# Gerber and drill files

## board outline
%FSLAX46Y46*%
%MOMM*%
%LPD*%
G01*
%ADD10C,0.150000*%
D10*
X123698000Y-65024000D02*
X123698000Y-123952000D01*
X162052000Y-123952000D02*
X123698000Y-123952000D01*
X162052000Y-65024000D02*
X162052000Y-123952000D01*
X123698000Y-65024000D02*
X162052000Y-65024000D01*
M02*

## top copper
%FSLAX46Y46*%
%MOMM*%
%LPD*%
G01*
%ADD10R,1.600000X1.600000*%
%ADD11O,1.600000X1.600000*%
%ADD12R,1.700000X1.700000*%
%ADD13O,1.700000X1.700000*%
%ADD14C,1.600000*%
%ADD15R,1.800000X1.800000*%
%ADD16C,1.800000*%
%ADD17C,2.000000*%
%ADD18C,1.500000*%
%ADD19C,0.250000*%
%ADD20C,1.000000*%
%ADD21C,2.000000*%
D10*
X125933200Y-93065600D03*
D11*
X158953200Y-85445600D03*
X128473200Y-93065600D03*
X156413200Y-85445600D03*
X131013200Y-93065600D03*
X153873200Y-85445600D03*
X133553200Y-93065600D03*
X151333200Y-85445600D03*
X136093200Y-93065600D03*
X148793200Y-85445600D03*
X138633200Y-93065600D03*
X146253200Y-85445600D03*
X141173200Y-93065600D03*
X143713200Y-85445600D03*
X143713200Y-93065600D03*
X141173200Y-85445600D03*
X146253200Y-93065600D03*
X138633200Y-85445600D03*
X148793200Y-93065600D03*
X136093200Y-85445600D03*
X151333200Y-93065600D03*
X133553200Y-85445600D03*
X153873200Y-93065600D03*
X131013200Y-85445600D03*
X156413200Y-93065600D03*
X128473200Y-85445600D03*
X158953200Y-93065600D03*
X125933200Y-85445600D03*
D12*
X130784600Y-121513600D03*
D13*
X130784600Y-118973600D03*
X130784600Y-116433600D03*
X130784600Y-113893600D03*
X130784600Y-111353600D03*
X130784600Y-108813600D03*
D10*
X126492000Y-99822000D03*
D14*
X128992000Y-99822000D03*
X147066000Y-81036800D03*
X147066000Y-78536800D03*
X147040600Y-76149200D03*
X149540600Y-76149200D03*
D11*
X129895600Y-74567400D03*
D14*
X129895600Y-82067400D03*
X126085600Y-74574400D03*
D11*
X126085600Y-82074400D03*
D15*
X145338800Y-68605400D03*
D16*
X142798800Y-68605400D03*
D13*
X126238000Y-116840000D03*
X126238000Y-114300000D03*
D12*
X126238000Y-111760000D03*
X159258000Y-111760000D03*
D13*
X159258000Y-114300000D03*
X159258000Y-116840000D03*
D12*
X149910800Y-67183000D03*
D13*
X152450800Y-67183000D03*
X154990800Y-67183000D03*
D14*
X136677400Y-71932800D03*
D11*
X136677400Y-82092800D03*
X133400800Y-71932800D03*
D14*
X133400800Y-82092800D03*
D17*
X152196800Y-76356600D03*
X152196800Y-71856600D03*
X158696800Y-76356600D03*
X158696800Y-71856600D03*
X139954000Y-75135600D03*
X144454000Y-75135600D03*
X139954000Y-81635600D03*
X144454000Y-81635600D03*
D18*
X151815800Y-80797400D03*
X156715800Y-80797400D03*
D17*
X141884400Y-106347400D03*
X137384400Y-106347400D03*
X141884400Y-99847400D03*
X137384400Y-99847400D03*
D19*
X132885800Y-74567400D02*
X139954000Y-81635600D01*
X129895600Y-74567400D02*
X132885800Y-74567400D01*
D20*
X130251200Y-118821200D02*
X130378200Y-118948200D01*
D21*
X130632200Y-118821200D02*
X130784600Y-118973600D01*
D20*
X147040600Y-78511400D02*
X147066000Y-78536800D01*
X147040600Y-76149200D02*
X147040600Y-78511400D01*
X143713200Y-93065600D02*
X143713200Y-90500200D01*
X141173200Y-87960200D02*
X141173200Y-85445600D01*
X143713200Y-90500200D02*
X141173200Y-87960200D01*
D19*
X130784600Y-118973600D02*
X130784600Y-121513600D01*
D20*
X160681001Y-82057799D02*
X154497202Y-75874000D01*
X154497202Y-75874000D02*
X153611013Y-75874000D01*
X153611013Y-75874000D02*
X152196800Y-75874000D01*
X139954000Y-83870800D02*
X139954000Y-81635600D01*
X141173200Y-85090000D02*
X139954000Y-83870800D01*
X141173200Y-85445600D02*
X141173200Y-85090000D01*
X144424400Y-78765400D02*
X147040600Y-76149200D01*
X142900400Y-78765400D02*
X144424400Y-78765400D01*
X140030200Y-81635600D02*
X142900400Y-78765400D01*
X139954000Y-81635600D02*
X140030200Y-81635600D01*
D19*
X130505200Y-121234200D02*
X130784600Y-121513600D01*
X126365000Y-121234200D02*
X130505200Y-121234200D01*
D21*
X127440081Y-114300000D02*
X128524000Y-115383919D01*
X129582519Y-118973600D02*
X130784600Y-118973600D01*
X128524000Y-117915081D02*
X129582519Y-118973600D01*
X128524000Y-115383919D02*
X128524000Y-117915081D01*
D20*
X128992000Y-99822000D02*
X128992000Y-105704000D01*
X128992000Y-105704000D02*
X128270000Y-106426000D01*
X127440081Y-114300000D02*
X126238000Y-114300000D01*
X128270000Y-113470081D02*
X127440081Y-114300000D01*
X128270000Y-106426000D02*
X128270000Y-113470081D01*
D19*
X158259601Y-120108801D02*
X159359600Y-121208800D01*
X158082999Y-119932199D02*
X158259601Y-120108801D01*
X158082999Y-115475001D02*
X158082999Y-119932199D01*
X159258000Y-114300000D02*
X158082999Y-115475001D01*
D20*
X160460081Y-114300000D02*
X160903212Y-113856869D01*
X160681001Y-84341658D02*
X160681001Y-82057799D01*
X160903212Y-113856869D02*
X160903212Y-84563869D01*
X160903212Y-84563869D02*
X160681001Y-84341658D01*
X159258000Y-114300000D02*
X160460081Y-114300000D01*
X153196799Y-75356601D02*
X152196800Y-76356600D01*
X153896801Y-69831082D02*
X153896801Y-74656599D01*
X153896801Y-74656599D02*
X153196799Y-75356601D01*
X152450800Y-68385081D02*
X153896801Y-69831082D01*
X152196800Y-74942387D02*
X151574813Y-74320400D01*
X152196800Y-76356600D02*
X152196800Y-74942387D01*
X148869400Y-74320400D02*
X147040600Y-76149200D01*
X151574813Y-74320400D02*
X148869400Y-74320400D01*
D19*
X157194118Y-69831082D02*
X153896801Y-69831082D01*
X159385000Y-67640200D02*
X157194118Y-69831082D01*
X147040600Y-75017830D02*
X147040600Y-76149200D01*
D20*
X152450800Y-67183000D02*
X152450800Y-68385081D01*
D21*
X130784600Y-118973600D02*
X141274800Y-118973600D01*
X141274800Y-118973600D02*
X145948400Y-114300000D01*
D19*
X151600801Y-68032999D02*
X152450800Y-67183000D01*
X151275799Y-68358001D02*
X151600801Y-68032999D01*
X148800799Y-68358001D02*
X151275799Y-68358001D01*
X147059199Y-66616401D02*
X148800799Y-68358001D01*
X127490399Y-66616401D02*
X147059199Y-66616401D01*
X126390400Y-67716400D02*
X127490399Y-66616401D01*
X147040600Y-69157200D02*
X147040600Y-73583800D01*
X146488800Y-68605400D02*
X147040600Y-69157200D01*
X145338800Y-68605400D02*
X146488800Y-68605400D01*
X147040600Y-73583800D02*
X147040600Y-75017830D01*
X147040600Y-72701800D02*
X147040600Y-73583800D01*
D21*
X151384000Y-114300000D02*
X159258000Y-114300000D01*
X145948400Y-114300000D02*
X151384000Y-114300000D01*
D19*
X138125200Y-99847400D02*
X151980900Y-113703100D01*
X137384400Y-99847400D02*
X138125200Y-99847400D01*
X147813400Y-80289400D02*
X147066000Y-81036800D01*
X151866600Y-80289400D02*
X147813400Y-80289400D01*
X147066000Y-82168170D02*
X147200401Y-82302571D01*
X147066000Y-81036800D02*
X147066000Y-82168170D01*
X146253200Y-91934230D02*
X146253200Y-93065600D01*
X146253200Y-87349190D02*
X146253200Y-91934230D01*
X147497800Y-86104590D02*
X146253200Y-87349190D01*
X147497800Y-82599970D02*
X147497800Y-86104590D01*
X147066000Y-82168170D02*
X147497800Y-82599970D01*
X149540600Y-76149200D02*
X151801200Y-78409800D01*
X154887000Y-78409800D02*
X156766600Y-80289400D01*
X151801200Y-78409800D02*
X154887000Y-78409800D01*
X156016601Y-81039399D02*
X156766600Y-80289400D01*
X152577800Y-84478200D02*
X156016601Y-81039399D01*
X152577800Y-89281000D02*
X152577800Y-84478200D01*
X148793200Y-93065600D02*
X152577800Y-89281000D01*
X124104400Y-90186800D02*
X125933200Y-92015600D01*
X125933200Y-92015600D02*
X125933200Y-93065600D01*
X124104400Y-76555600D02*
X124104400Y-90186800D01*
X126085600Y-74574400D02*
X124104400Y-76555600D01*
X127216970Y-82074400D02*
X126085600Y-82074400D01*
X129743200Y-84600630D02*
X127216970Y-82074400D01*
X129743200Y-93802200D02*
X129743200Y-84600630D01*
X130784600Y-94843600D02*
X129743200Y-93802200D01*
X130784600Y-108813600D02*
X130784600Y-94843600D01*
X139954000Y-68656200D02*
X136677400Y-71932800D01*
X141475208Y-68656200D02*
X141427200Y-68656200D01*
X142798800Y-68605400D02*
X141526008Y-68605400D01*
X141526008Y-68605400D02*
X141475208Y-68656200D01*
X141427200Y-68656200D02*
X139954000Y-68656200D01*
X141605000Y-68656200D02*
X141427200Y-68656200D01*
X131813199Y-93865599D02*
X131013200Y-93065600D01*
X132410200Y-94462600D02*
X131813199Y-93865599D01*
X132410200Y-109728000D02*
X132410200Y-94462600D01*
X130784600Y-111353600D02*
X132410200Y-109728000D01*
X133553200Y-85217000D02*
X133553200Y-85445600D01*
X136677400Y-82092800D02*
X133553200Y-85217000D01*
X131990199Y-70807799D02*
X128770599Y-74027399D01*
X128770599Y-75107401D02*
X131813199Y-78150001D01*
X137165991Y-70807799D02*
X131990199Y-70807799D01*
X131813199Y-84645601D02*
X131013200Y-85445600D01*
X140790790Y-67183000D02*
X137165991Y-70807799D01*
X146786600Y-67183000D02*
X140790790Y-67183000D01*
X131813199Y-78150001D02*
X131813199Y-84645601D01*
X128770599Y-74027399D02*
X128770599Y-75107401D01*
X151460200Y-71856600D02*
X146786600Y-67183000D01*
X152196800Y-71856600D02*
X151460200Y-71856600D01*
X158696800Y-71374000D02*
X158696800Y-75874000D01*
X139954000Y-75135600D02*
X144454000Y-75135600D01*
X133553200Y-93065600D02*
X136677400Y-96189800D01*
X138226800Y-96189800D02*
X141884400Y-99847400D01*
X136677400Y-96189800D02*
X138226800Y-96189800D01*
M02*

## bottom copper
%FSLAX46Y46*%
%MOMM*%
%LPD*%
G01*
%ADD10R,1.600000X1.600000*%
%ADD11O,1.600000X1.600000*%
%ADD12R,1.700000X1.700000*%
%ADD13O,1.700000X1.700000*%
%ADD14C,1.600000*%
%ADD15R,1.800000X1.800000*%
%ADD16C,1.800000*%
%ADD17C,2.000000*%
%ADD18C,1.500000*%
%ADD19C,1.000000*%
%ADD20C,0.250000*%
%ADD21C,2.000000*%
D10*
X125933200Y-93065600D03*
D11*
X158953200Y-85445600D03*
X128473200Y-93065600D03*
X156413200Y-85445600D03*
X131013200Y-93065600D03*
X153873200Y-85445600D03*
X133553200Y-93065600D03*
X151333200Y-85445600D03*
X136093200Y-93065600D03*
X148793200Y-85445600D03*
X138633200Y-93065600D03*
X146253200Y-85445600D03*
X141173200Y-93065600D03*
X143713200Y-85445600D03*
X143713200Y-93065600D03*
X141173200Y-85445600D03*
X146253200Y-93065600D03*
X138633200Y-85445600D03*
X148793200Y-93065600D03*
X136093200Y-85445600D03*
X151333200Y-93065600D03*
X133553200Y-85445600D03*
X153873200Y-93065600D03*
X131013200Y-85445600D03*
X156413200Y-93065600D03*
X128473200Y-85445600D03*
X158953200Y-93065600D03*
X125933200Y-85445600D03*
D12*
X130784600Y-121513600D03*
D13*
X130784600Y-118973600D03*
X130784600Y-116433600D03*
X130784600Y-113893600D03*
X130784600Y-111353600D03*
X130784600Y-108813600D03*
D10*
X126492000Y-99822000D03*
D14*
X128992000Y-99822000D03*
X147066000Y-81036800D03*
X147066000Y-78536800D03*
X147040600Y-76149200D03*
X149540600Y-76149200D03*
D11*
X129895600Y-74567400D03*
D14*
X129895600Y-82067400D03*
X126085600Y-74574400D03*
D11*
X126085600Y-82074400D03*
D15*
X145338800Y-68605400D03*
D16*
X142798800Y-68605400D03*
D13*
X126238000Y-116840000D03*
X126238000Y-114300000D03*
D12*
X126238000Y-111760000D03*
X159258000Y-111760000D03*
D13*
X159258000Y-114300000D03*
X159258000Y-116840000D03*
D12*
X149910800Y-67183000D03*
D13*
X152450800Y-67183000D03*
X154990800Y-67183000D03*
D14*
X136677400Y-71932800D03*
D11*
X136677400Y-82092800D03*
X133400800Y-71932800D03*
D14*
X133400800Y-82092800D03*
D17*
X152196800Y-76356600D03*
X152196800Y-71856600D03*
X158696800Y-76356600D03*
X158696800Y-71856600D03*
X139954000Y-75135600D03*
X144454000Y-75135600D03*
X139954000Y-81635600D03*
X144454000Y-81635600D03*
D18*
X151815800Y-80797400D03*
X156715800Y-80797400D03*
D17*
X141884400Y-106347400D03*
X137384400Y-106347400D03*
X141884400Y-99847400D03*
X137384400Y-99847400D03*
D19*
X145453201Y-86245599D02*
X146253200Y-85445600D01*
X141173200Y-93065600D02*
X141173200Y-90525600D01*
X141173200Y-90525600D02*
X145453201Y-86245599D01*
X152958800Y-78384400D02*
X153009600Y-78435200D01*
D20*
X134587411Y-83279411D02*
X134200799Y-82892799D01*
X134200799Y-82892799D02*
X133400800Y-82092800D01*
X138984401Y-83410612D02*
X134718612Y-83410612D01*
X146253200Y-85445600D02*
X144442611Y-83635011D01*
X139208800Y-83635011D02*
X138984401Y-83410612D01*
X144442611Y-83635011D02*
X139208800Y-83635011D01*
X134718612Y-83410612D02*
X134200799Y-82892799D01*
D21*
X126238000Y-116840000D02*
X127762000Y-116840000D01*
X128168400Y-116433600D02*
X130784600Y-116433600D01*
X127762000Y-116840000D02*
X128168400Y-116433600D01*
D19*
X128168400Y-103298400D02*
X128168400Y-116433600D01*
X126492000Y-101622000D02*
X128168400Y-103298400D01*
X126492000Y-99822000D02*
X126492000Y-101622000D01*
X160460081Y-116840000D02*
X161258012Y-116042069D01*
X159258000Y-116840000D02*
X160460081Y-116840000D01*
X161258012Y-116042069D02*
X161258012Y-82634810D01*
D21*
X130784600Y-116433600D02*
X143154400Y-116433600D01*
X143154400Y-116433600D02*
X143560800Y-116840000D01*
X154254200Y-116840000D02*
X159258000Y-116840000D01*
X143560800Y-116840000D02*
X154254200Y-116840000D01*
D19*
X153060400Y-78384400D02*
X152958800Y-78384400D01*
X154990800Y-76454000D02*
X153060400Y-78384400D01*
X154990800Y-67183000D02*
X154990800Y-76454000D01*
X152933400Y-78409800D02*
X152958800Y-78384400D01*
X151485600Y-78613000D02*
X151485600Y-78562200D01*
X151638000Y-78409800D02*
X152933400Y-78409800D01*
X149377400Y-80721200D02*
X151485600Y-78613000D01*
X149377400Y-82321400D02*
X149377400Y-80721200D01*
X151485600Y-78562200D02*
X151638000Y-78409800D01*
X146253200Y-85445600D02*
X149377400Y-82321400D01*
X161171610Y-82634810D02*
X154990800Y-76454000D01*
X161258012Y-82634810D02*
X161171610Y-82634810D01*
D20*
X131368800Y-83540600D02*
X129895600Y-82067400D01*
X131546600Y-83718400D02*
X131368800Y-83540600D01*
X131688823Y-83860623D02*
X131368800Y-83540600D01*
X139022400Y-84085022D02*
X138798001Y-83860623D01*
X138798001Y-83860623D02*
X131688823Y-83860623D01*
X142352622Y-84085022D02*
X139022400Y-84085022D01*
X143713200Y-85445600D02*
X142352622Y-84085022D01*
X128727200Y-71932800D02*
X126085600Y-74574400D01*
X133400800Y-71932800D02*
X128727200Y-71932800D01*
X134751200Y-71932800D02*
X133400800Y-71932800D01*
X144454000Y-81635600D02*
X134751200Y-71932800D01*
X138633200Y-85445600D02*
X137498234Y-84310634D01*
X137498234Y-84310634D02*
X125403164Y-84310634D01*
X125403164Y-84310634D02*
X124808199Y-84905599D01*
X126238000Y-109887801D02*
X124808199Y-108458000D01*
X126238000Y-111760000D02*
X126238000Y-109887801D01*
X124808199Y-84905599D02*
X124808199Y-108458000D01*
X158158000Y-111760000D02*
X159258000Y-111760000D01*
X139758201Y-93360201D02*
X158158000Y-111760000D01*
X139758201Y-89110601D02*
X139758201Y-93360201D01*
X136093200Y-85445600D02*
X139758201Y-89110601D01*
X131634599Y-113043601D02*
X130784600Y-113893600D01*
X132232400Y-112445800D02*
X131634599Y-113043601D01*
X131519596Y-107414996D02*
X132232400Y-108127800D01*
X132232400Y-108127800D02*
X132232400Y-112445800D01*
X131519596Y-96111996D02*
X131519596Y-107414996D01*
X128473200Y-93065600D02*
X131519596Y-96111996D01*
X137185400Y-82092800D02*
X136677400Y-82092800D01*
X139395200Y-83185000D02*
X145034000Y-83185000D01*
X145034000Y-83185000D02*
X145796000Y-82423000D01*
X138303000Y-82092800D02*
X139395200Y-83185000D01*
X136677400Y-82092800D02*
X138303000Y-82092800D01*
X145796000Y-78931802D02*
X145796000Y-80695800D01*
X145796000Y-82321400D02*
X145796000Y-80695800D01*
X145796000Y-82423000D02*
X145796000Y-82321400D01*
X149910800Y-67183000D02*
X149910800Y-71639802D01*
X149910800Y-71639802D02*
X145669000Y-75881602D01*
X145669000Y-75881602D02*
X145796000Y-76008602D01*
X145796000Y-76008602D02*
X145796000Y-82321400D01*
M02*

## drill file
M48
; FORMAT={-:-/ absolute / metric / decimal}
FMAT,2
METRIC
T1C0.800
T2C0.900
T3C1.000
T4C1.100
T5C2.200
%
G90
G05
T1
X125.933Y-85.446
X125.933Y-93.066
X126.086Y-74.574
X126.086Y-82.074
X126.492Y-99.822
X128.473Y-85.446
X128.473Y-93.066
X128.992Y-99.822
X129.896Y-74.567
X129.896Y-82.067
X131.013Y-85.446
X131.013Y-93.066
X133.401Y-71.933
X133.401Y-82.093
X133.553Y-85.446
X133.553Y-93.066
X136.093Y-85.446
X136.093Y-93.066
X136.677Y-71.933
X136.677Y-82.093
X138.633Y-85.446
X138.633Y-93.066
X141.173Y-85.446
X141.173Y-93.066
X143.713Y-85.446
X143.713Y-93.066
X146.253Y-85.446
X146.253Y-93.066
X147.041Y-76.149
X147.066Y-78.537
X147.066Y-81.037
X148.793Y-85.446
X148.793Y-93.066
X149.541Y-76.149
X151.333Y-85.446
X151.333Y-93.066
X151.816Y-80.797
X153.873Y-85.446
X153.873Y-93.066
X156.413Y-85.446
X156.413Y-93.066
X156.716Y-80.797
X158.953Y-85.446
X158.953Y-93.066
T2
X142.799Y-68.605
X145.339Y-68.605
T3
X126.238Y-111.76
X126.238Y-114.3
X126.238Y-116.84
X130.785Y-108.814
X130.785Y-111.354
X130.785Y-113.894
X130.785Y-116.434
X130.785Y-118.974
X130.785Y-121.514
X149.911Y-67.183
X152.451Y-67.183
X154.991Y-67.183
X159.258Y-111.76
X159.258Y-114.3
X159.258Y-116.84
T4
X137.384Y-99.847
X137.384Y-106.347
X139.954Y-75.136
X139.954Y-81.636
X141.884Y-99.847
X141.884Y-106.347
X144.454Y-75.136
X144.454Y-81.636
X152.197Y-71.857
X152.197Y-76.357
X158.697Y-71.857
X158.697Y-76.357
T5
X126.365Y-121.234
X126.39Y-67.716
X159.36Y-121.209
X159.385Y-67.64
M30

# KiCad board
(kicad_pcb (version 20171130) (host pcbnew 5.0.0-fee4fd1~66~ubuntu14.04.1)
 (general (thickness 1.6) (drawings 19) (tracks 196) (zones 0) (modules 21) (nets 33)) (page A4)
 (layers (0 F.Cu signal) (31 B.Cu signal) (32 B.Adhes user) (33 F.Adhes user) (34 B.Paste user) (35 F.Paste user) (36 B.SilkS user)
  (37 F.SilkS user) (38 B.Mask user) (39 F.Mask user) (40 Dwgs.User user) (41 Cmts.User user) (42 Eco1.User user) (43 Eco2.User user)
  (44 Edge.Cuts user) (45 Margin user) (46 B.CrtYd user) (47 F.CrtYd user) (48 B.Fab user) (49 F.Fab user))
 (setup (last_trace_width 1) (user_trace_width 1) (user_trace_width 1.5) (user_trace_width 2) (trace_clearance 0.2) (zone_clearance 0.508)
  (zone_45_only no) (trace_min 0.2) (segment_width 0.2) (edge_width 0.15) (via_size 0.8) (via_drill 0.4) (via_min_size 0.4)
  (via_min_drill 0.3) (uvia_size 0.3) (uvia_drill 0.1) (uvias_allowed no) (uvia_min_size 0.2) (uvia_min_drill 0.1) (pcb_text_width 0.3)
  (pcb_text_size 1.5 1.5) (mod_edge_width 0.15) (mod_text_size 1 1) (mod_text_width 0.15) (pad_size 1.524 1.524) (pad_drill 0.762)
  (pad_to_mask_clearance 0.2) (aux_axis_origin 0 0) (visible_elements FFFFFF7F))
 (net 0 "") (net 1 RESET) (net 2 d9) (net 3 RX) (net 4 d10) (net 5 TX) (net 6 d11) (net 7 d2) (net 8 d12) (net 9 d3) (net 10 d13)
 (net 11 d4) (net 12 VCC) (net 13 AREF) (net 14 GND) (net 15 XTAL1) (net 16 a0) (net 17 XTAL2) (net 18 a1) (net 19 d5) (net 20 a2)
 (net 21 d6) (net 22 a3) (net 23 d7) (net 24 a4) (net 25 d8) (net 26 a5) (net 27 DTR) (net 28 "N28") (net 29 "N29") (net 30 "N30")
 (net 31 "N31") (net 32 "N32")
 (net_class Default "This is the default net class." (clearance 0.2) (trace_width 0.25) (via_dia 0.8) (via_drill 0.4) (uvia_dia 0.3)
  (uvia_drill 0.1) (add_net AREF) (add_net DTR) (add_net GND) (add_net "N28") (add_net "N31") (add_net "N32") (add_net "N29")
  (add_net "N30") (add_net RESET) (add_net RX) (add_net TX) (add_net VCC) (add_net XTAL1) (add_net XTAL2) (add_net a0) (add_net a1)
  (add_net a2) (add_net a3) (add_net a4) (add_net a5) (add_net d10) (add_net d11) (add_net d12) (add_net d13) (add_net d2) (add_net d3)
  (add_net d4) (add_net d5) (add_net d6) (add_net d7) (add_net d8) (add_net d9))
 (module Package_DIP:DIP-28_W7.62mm (layer F.Cu) (at 125.9332 93.0656 90)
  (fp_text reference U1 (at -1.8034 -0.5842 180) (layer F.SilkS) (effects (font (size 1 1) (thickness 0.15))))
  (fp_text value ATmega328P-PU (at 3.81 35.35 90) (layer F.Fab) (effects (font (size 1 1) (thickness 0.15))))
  (pad 1 thru_hole rect (at 0 0 90) (size 1.6 1.6) (drill 0.8) (layers *.Cu *.Mask) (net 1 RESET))
  (pad 15 thru_hole oval (at 7.62 33.02 90) (size 1.6 1.6) (drill 0.8) (layers *.Cu *.Mask) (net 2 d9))
  (pad 2 thru_hole oval (at 0 2.54 90) (size 1.6 1.6) (drill 0.8) (layers *.Cu *.Mask) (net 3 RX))
  (pad 16 thru_hole oval (at 7.62 30.48 90) (size 1.6 1.6) (drill 0.8) (layers *.Cu *.Mask) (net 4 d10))
  (pad 3 thru_hole oval (at 0 5.08 90) (size 1.6 1.6) (drill 0.8) (layers *.Cu *.Mask) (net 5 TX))
  (pad 17 thru_hole oval (at 7.62 27.94 90) (size 1.6 1.6) (drill 0.8) (layers *.Cu *.Mask) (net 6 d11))
  (pad 4 thru_hole oval (at 0 7.62 90) (size 1.6 1.6) (drill 0.8) (layers *.Cu *.Mask) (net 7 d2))
  (pad 18 thru_hole oval (at 7.62 25.4 90) (size 1.6 1.6) (drill 0.8) (layers *.Cu *.Mask) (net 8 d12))
  (pad 5 thru_hole oval (at 0 10.16 90) (size 1.6 1.6) (drill 0.8) (layers *.Cu *.Mask) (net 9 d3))
  (pad 19 thru_hole oval (at 7.62 22.86 90) (size 1.6 1.6) (drill 0.8) (layers *.Cu *.Mask) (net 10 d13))
  (pad 6 thru_hole oval (at 0 12.7 90) (size 1.6 1.6) (drill 0.8) (layers *.Cu *.Mask) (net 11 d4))
  (pad 20 thru_hole oval (at 7.62 20.32 90) (size 1.6 1.6) (drill 0.8) (layers *.Cu *.Mask) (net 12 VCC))
  (pad 7 thru_hole oval (at 0 15.24 90) (size 1.6 1.6) (drill 0.8) (layers *.Cu *.Mask) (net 12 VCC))
  (pad 21 thru_hole oval (at 7.62 17.78 90) (size 1.6 1.6) (drill 0.8) (layers *.Cu *.Mask) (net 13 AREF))
  (pad 8 thru_hole oval (at 0 17.78 90) (size 1.6 1.6) (drill 0.8) (layers *.Cu *.Mask) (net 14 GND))
  (pad 22 thru_hole oval (at 7.62 15.24 90) (size 1.6 1.6) (drill 0.8) (layers *.Cu *.Mask) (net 14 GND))
  (pad 9 thru_hole oval (at 0 20.32 90) (size 1.6 1.6) (drill 0.8) (layers *.Cu *.Mask) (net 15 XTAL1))
  (pad 23 thru_hole oval (at 7.62 12.7 90) (size 1.6 1.6) (drill 0.8) (layers *.Cu *.Mask) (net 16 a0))
  (pad 10 thru_hole oval (at 0 22.86 90) (size 1.6 1.6) (drill 0.8) (layers *.Cu *.Mask) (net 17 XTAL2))
  (pad 24 thru_hole oval (at 7.62 10.16 90) (size 1.6 1.6) (drill 0.8) (layers *.Cu *.Mask) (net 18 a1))
  (pad 11 thru_hole oval (at 0 25.4 90) (size 1.6 1.6) (drill 0.8) (layers *.Cu *.Mask) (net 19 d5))
  (pad 25 thru_hole oval (at 7.62 7.62 90) (size 1.6 1.6) (drill 0.8) (layers *.Cu *.Mask) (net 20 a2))
  (pad 12 thru_hole oval (at 0 27.94 90) (size 1.6 1.6) (drill 0.8) (layers *.Cu *.Mask) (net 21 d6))
  (pad 26 thru_hole oval (at 7.62 5.08 90) (size 1.6 1.6) (drill 0.8) (layers *.Cu *.Mask) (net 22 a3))
  (pad 13 thru_hole oval (at 0 30.48 90) (size 1.6 1.6) (drill 0.8) (layers *.Cu *.Mask) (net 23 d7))
  (pad 27 thru_hole oval (at 7.62 2.54 90) (size 1.6 1.6) (drill 0.8) (layers *.Cu *.Mask) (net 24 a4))
  (pad 14 thru_hole oval (at 0 33.02 90) (size 1.6 1.6) (drill 0.8) (layers *.Cu *.Mask) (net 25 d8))
  (pad 28 thru_hole oval (at 7.62 0 90) (size 1.6 1.6) (drill 0.8) (layers *.Cu *.Mask) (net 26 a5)))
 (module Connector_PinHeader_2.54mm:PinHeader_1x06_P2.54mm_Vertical (layer F.Cu) (at 130.7846 121.5136 180)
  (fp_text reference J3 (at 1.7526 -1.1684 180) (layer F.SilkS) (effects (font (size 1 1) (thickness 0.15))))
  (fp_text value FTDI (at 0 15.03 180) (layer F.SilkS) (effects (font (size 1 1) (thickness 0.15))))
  (pad 1 thru_hole rect (at 0 0 180) (size 1.7 1.7) (drill 1) (layers *.Cu *.Mask) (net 14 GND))
  (pad 2 thru_hole oval (at 0 2.54 180) (size 1.7 1.7) (drill 1) (layers *.Cu *.Mask) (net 14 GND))
  (pad 3 thru_hole oval (at 0 5.08 180) (size 1.7 1.7) (drill 1) (layers *.Cu *.Mask) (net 12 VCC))
  (pad 4 thru_hole oval (at 0 7.62 180) (size 1.7 1.7) (drill 1) (layers *.Cu *.Mask) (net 3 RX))
  (pad 5 thru_hole oval (at 0 10.16 180) (size 1.7 1.7) (drill 1) (layers *.Cu *.Mask) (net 5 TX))
  (pad 6 thru_hole oval (at 0 12.7 180) (size 1.7 1.7) (drill 1) (layers *.Cu *.Mask) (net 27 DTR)))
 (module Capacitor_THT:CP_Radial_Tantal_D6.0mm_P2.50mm (layer F.Cu) (at 126.492 99.822)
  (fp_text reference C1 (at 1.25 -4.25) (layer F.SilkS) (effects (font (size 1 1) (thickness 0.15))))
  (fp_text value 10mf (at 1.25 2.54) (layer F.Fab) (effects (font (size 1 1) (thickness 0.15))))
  (pad 1 thru_hole rect (at 0 0) (size 1.6 1.6) (drill 0.8) (layers *.Cu *.Mask) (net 12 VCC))
  (pad 2 thru_hole circle (at 2.5 0) (size 1.6 1.6) (drill 0.8) (layers *.Cu *.Mask) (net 14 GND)))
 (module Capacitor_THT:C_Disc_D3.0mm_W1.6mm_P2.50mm (layer F.Cu) (at 147.066 78.5368 270)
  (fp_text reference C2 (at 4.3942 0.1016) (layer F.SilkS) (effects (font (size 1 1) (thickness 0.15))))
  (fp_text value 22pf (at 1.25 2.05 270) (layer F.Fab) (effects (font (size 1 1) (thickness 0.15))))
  (pad 2 thru_hole circle (at 2.5 0 270) (size 1.6 1.6) (drill 0.8) (layers *.Cu *.Mask) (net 15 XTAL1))
  (pad 1 thru_hole circle (at 0 0 270) (size 1.6 1.6) (drill 0.8) (layers *.Cu *.Mask) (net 14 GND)))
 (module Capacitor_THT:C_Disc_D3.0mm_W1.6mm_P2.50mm (layer F.Cu) (at 147.0406 76.1492)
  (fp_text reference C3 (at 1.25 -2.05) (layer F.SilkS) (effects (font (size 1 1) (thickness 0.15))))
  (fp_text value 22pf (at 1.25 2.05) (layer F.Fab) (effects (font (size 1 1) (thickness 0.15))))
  (pad 1 thru_hole circle (at 0 0) (size 1.6 1.6) (drill 0.8) (layers *.Cu *.Mask) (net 14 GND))
  (pad 2 thru_hole circle (at 2.5 0) (size 1.6 1.6) (drill 0.8) (layers *.Cu *.Mask) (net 17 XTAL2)))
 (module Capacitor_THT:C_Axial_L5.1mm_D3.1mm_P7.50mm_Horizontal (layer F.Cu) (at 129.8956 82.0674 90)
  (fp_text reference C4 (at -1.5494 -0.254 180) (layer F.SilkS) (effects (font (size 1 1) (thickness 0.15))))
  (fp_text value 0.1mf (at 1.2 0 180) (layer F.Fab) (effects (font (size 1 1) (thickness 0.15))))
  (pad 2 thru_hole oval (at 7.5 0 90) (size 1.6 1.6) (drill 0.8) (layers *.Cu *.Mask) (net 14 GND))
  (pad 1 thru_hole circle (at 0 0 90) (size 1.6 1.6) (drill 0.8) (layers *.Cu *.Mask) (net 13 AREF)))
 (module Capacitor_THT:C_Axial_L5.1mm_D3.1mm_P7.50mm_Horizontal (layer F.Cu) (at 126.0856 74.5744 270)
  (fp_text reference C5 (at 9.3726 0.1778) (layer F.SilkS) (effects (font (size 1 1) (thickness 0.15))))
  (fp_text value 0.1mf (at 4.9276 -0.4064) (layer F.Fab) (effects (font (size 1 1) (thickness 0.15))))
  (pad 1 thru_hole circle (at 0 0 270) (size 1.6 1.6) (drill 0.8) (layers *.Cu *.Mask) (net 1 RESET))
  (pad 2 thru_hole oval (at 7.5 0 270) (size 1.6 1.6) (drill 0.8) (layers *.Cu *.Mask) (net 27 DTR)))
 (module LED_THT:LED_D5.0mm (layer F.Cu) (at 145.3388 68.6054 180)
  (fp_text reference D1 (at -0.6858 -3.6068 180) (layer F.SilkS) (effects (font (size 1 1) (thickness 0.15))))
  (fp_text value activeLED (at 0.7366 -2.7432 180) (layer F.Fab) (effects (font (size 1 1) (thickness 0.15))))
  (pad 1 thru_hole rect (at 0 0 180) (size 1.8 1.8) (drill 0.9) (layers *.Cu *.Mask) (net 14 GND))
  (pad 2 thru_hole circle (at 2.54 0 180) (size 1.8 1.8) (drill 0.9) (layers *.Cu *.Mask) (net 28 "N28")))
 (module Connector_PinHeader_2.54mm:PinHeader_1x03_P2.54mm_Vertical (layer F.Cu) (at 126.238 111.76)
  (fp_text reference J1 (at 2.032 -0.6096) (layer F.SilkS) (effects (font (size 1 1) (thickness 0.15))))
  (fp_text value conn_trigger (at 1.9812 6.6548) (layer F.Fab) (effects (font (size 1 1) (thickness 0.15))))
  (pad 3 thru_hole oval (at 0 5.08) (size 1.7 1.7) (drill 1) (layers *.Cu *.Mask) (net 12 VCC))
  (pad 2 thru_hole oval (at 0 2.54) (size 1.7 1.7) (drill 1) (layers *.Cu *.Mask) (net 14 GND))
  (pad 1 thru_hole rect (at 0 0) (size 1.7 1.7) (drill 1) (layers *.Cu *.Mask) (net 16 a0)))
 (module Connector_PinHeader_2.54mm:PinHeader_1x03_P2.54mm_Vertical (layer F.Cu) (at 159.258 111.76)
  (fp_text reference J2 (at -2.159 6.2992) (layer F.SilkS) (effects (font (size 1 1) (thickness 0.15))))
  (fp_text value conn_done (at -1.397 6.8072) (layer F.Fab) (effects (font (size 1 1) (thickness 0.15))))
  (pad 1 thru_hole rect (at 0 0) (size 1.7 1.7) (drill 1) (layers *.Cu *.Mask) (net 18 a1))
  (pad 2 thru_hole oval (at 0 2.54) (size 1.7 1.7) (drill 1) (layers *.Cu *.Mask) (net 14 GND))
  (pad 3 thru_hole oval (at 0 5.08) (size 1.7 1.7) (drill 1) (layers *.Cu *.Mask) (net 12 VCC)))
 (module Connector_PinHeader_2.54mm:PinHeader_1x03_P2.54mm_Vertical (layer F.Cu) (at 149.9108 67.183 90)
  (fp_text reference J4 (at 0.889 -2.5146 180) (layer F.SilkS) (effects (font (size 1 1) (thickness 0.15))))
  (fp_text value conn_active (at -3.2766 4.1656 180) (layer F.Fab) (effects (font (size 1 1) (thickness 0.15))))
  (pad 1 thru_hole rect (at 0 0 90) (size 1.7 1.7) (drill 1) (layers *.Cu *.Mask) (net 20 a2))
  (pad 2 thru_hole oval (at 0 2.54 90) (size 1.7 1.7) (drill 1) (layers *.Cu *.Mask) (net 14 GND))
  (pad 3 thru_hole oval (at 0 5.08 90) (size 1.7 1.7) (drill 1) (layers *.Cu *.Mask) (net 12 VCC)))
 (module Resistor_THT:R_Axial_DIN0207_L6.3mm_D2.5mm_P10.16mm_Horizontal (layer F.Cu) (at 136.6774 71.9328 270)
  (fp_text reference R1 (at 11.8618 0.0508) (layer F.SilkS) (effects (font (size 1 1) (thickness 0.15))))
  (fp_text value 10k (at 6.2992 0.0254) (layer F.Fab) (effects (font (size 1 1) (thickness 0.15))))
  (pad 1 thru_hole circle (at 0 0 270) (size 1.6 1.6) (drill 0.8) (layers *.Cu *.Mask) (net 28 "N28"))
  (pad 2 thru_hole oval (at 10.16 0 270) (size 1.6 1.6) (drill 0.8) (layers *.Cu *.Mask) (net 20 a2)))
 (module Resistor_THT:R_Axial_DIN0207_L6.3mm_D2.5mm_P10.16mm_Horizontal (layer F.Cu) (at 133.4008 82.0928 90)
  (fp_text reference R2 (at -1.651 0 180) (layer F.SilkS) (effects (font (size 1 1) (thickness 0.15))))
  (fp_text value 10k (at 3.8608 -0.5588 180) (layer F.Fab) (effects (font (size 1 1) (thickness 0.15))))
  (pad 2 thru_hole oval (at 10.16 0 90) (size 1.6 1.6) (drill 0.8) (layers *.Cu *.Mask) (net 1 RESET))
  (pad 1 thru_hole circle (at 0 0 90) (size 1.6 1.6) (drill 0.8) (layers *.Cu *.Mask) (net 12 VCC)))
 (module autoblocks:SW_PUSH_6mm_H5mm (layer F.Cu) (at 152.1968 71.8566)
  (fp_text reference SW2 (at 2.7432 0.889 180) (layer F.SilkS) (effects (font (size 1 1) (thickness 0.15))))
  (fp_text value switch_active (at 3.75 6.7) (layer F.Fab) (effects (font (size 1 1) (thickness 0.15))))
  (pad 2 thru_hole circle (at 0 4.5 90) (size 2 2) (drill 1.1) (layers *.Cu *.Mask) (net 14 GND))
  (pad 1 thru_hole circle (at 0 0 90) (size 2 2) (drill 1.1) (layers *.Cu *.Mask) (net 22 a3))
  (pad 4 thru_hole circle (at 6.5 4.5 90) (size 2 2) (drill 1.1) (layers *.Cu *.Mask) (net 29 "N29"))
  (pad 3 thru_hole circle (at 6.5 0 90) (size 2 2) (drill 1.1) (layers *.Cu *.Mask) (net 29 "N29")))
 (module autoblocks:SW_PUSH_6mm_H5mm (layer F.Cu) (at 139.954 81.6356 90)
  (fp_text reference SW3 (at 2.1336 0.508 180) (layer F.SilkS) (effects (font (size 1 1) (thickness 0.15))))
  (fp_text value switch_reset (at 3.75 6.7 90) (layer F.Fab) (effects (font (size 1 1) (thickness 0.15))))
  (pad 3 thru_hole circle (at 6.5 0 180) (size 2 2) (drill 1.1) (layers *.Cu *.Mask) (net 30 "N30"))
  (pad 4 thru_hole circle (at 6.5 4.5 180) (size 2 2) (drill 1.1) (layers *.Cu *.Mask) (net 30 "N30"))
  (pad 1 thru_hole circle (at 0 0 180) (size 2 2) (drill 1.1) (layers *.Cu *.Mask) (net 14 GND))
  (pad 2 thru_hole circle (at 0 4.5 180) (size 2 2) (drill 1.1) (layers *.Cu *.Mask) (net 1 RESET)))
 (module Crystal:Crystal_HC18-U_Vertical (layer F.Cu) (at 151.8158 80.7974)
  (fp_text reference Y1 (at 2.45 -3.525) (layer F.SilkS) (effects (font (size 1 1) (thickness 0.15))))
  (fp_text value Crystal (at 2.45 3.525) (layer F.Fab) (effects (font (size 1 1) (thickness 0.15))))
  (pad 1 thru_hole circle (at 0 0) (size 1.5 1.5) (drill 0.8) (layers *.Cu *.Mask) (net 15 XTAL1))
  (pad 2 thru_hole circle (at 4.9 0) (size 1.5 1.5) (drill 0.8) (layers *.Cu *.Mask) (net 17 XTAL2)))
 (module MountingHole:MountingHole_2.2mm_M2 (layer F.Cu) (at 126.365 121.2342)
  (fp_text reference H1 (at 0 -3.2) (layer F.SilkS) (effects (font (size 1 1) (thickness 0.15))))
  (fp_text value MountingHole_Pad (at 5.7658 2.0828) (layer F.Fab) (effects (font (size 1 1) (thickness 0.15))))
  (pad 1 np_thru_hole circle (at 0 0) (size 2.2 2.2) (drill 2.2) (layers *.Cu *.Mask) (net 14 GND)))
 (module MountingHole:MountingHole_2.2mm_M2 (layer F.Cu) (at 159.3596 121.2088)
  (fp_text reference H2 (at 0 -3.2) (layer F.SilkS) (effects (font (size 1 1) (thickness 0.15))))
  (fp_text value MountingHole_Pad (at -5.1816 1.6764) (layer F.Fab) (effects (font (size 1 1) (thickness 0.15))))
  (pad 1 np_thru_hole circle (at 0 0) (size 2.2 2.2) (drill 2.2) (layers *.Cu *.Mask) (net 14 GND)))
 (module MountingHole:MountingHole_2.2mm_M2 (layer F.Cu) (at 159.385 67.6402)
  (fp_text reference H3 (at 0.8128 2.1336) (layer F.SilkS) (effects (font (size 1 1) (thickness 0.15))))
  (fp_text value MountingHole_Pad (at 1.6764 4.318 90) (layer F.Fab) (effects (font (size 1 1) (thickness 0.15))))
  (pad 1 np_thru_hole circle (at 0 0) (size 2.2 2.2) (drill 2.2) (layers *.Cu *.Mask) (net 14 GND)))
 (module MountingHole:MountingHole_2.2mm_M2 (layer F.Cu) (at 126.3904 67.7164)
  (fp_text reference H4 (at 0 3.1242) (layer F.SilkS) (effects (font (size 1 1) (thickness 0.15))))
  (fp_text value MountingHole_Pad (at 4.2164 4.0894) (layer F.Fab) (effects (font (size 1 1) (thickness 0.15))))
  (pad 1 np_thru_hole circle (at 0 0) (size 2.2 2.2) (drill 2.2) (layers *.Cu *.Mask) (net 14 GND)))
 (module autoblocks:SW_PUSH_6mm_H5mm (layer F.Cu) (at 141.8844 99.8474 270)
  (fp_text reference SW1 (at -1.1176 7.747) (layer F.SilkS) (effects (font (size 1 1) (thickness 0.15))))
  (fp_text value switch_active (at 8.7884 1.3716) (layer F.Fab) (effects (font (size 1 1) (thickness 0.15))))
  (pad 3 thru_hole circle (at 6.5 0) (size 2 2) (drill 1.1) (layers *.Cu *.Mask) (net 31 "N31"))
  (pad 4 thru_hole circle (at 6.5 4.5) (size 2 2) (drill 1.1) (layers *.Cu *.Mask) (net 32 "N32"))
  (pad 1 thru_hole circle (at 0 0) (size 2 2) (drill 1.1) (layers *.Cu *.Mask) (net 7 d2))
  (pad 2 thru_hole circle (at 0 4.5) (size 2 2) (drill 1.1) (layers *.Cu *.Mask) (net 14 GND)))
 (gr_line (start 123.698 65.024) (end 123.698 123.952) (layer Edge.Cuts) (width 0.15))
 (gr_line (start 162.052 123.952) (end 123.698 123.952) (layer Edge.Cuts) (width 0.15))
 (gr_line (start 162.052 65.024) (end 162.052 123.952) (layer Edge.Cuts) (width 0.15))
 (gr_line (start 123.698 65.024) (end 162.052 65.024) (layer Edge.Cuts) (width 0.15))
 (segment (start 132.8858 74.5674) (end 139.954 81.6356) (width 0.25) (layer F.Cu) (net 14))
 (segment (start 129.8956 74.5674) (end 132.8858 74.5674) (width 0.25) (layer F.Cu) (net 14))
 (segment (start 130.2512 118.8212) (end 130.3782 118.9482) (width 1) (layer F.Cu) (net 14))
 (segment (start 130.6322 118.8212) (end 130.7846 118.9736) (width 2) (layer F.Cu) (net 14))
 (segment (start 147.0406 78.5114) (end 147.066 78.5368) (width 1) (layer F.Cu) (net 14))
 (segment (start 147.0406 76.1492) (end 147.0406 78.5114) (width 1) (layer F.Cu) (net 14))
 (segment (start 143.7132 93.0656) (end 143.7132 90.5002) (width 1) (layer F.Cu) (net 14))
 (segment (start 141.1732 87.9602) (end 141.1732 85.4456) (width 1) (layer F.Cu) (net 14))
 (segment (start 143.7132 90.5002) (end 141.1732 87.9602) (width 1) (layer F.Cu) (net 14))
 (segment (start 130.7846 118.9736) (end 130.7846 121.5136) (width 0.25) (layer F.Cu) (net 14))
 (segment (start 160.681001 82.057799) (end 154.497202 75.874) (width 1) (layer F.Cu) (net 14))
 (segment (start 154.497202 75.874) (end 153.611013 75.874) (width 1) (layer F.Cu) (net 14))
 (segment (start 153.611013 75.874) (end 152.1968 75.874) (width 1) (layer F.Cu) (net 14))
 (segment (start 139.954 83.8708) (end 139.954 81.6356) (width 1) (layer F.Cu) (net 14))
 (segment (start 141.1732 85.09) (end 139.954 83.8708) (width 1) (layer F.Cu) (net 14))
 (segment (start 141.1732 85.4456) (end 141.1732 85.09) (width 1) (layer F.Cu) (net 14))
 (segment (start 144.4244 78.7654) (end 147.0406 76.1492) (width 1) (layer F.Cu) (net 14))
 (segment (start 142.9004 78.7654) (end 144.4244 78.7654) (width 1) (layer F.Cu) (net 14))
 (segment (start 140.0302 81.6356) (end 142.9004 78.7654) (width 1) (layer F.Cu) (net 14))
 (segment (start 139.954 81.6356) (end 140.0302 81.6356) (width 1) (layer F.Cu) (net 14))
 (segment (start 130.5052 121.2342) (end 130.7846 121.5136) (width 0.25) (layer F.Cu) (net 14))
 (segment (start 126.365 121.2342) (end 130.5052 121.2342) (width 0.25) (layer F.Cu) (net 14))
 (segment (start 127.440081 114.3) (end 128.524 115.383919) (width 2) (layer F.Cu) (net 14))
 (segment (start 129.582519 118.9736) (end 130.7846 118.9736) (width 2) (layer F.Cu) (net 14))
 (segment (start 128.524 117.915081) (end 129.582519 118.9736) (width 2) (layer F.Cu) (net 14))
 (segment (start 128.524 115.383919) (end 128.524 117.915081) (width 2) (layer F.Cu) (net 14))
 (segment (start 128.992 99.822) (end 128.992 105.704) (width 1) (layer F.Cu) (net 14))
 (segment (start 128.992 105.704) (end 128.27 106.426) (width 1) (layer F.Cu) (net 14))
 (segment (start 127.440081 114.3) (end 126.238 114.3) (width 1) (layer F.Cu) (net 14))
 (segment (start 128.27 113.470081) (end 127.440081 114.3) (width 1) (layer F.Cu) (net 14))
 (segment (start 128.27 106.426) (end 128.27 113.470081) (width 1) (layer F.Cu) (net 14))
 (segment (start 158.259601 120.108801) (end 159.3596 121.2088) (width 0.25) (layer F.Cu) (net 14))
 (segment (start 158.082999 119.932199) (end 158.259601 120.108801) (width 0.25) (layer F.Cu) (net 14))
 (segment (start 158.082999 115.475001) (end 158.082999 119.932199) (width 0.25) (layer F.Cu) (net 14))
 (segment (start 159.258 114.3) (end 158.082999 115.475001) (width 0.25) (layer F.Cu) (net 14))
 (segment (start 160.460081 114.3) (end 160.903212 113.856869) (width 1) (layer F.Cu) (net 14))
 (segment (start 160.681001 84.341658) (end 160.681001 82.057799) (width 1) (layer F.Cu) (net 14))
 (segment (start 160.903212 113.856869) (end 160.903212 84.563869) (width 1) (layer F.Cu) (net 14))
 (segment (start 160.903212 84.563869) (end 160.681001 84.341658) (width 1) (layer F.Cu) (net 14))
 (segment (start 159.258 114.3) (end 160.460081 114.3) (width 1) (layer F.Cu) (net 14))
 (segment (start 153.196799 75.356601) (end 152.1968 76.3566) (width 1) (layer F.Cu) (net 14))
 (segment (start 153.896801 69.831082) (end 153.896801 74.656599) (width 1) (layer F.Cu) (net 14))
 (segment (start 153.896801 74.656599) (end 153.196799 75.356601) (width 1) (layer F.Cu) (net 14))
 (segment (start 152.4508 68.385081) (end 153.896801 69.831082) (width 1) (layer F.Cu) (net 14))
 (segment (start 152.1968 74.942387) (end 151.574813 74.3204) (width 1) (layer F.Cu) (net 14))
 (segment (start 152.1968 76.3566) (end 152.1968 74.942387) (width 1) (layer F.Cu) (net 14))
 (segment (start 148.8694 74.3204) (end 147.0406 76.1492) (width 1) (layer F.Cu) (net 14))
 (segment (start 151.574813 74.3204) (end 148.8694 74.3204) (width 1) (layer F.Cu) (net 14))
 (segment (start 157.194118 69.831082) (end 153.896801 69.831082) (width 0.25) (layer F.Cu) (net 14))
 (segment (start 159.385 67.6402) (end 157.194118 69.831082) (width 0.25) (layer F.Cu) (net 14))
 (segment (start 147.0406 75.01783) (end 147.0406 76.1492) (width 0.25) (layer F.Cu) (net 14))
 (segment (start 152.4508 67.183) (end 152.4508 68.385081) (width 1) (layer F.Cu) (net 14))
 (segment (start 130.7846 118.9736) (end 141.2748 118.9736) (width 2) (layer F.Cu) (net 14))
 (segment (start 141.2748 118.9736) (end 145.9484 114.3) (width 2) (layer F.Cu) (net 14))
 (segment (start 151.600801 68.032999) (end 152.4508 67.183) (width 0.25) (layer F.Cu) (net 14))
 (segment (start 151.275799 68.358001) (end 151.600801 68.032999) (width 0.25) (layer F.Cu) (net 14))
 (segment (start 148.800799 68.358001) (end 151.275799 68.358001) (width 0.25) (layer F.Cu) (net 14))
 (segment (start 147.059199 66.616401) (end 148.800799 68.358001) (width 0.25) (layer F.Cu) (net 14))
 (segment (start 127.490399 66.616401) (end 147.059199 66.616401) (width 0.25) (layer F.Cu) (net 14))
 (segment (start 126.3904 67.7164) (end 127.490399 66.616401) (width 0.25) (layer F.Cu) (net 14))
 (segment (start 147.0406 69.1572) (end 147.0406 73.5838) (width 0.25) (layer F.Cu) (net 14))
 (segment (start 146.4888 68.6054) (end 147.0406 69.1572) (width 0.25) (layer F.Cu) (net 14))
 (segment (start 145.3388 68.6054) (end 146.4888 68.6054) (width 0.25) (layer F.Cu) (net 14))
 (segment (start 147.0406 73.5838) (end 147.0406 75.01783) (width 0.25) (layer F.Cu) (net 14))
 (segment (start 147.0406 72.7018) (end 147.0406 73.5838) (width 0.25) (layer F.Cu) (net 14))
 (segment (start 151.384 114.3) (end 159.258 114.3) (width 2) (layer F.Cu) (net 14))
 (segment (start 145.9484 114.3) (end 151.384 114.3) (width 2) (layer F.Cu) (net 14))
 (segment (start 138.1252 99.8474) (end 151.9809 113.7031) (width 0.25) (layer F.Cu) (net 14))
 (segment (start 137.3844 99.8474) (end 138.1252 99.8474) (width 0.25) (layer F.Cu) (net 14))
 (segment (start 145.453201 86.245599) (end 146.2532 85.4456) (width 1) (layer B.Cu) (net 12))
 (segment (start 141.1732 93.0656) (end 141.1732 90.5256) (width 1) (layer B.Cu) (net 12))
 (segment (start 141.1732 90.5256) (end 145.453201 86.245599) (width 1) (layer B.Cu) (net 12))
 (segment (start 152.9588 78.3844) (end 153.0096 78.4352) (width 1) (layer B.Cu) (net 12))
 (segment (start 134.587411 83.279411) (end 134.200799 82.892799) (width 0.25) (layer B.Cu) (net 12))
 (segment (start 134.200799 82.892799) (end 133.4008 82.0928) (width 0.25) (layer B.Cu) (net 12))
 (segment (start 138.984401 83.410612) (end 134.718612 83.410612) (width 0.25) (layer B.Cu) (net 12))
 (segment (start 146.2532 85.4456) (end 144.442611 83.635011) (width 0.25) (layer B.Cu) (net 12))
 (segment (start 139.2088 83.635011) (end 138.984401 83.410612) (width 0.25) (layer B.Cu) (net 12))
 (segment (start 144.442611 83.635011) (end 139.2088 83.635011) (width 0.25) (layer B.Cu) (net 12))
 (segment (start 134.718612 83.410612) (end 134.200799 82.892799) (width 0.25) (layer B.Cu) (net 12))
 (segment (start 126.238 116.84) (end 127.762 116.84) (width 2) (layer B.Cu) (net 12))
 (segment (start 128.1684 116.4336) (end 130.7846 116.4336) (width 2) (layer B.Cu) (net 12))
 (segment (start 127.762 116.84) (end 128.1684 116.4336) (width 2) (layer B.Cu) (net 12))
 (segment (start 128.1684 103.2984) (end 128.1684 116.4336) (width 1) (layer B.Cu) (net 12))
 (segment (start 126.492 101.622) (end 128.1684 103.2984) (width 1) (layer B.Cu) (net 12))
 (segment (start 126.492 99.822) (end 126.492 101.622) (width 1) (layer B.Cu) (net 12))
 (segment (start 160.460081 116.84) (end 161.258012 116.042069) (width 1) (layer B.Cu) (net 12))
 (segment (start 159.258 116.84) (end 160.460081 116.84) (width 1) (layer B.Cu) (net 12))
 (segment (start 161.258012 116.042069) (end 161.258012 82.63481) (width 1) (layer B.Cu) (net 12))
 (segment (start 130.7846 116.4336) (end 143.1544 116.4336) (width 2) (layer B.Cu) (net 12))
 (segment (start 143.1544 116.4336) (end 143.5608 116.84) (width 2) (layer B.Cu) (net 12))
 (segment (start 154.2542 116.84) (end 159.258 116.84) (width 2) (layer B.Cu) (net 12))
 (segment (start 143.5608 116.84) (end 154.2542 116.84) (width 2) (layer B.Cu) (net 12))
 (segment (start 153.0604 78.3844) (end 152.9588 78.3844) (width 1) (layer B.Cu) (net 12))
 (segment (start 154.9908 76.454) (end 153.0604 78.3844) (width 1) (layer B.Cu) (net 12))
 (segment (start 154.9908 67.183) (end 154.9908 76.454) (width 1) (layer B.Cu) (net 12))
 (segment (start 152.9334 78.4098) (end 152.9588 78.3844) (width 1) (layer B.Cu) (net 12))
 (segment (start 151.4856 78.613) (end 151.4856 78.5622) (width 1) (layer B.Cu) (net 12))
 (segment (start 151.638 78.4098) (end 152.9334 78.4098) (width 1) (layer B.Cu) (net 12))
 (segment (start 149.3774 80.7212) (end 151.4856 78.613) (width 1) (layer B.Cu) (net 12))
 (segment (start 149.3774 82.3214) (end 149.3774 80.7212) (width 1) (layer B.Cu) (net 12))
 (segment (start 151.4856 78.5622) (end 151.638 78.4098) (width 1) (layer B.Cu) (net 12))
 (segment (start 146.2532 85.4456) (end 149.3774 82.3214) (width 1) (layer B.Cu) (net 12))
 (segment (start 161.17161 82.63481) (end 154.9908 76.454) (width 1) (layer B.Cu) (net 12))
 (segment (start 161.258012 82.63481) (end 161.17161 82.63481) (width 1) (layer B.Cu) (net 12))
 (segment (start 147.8134 80.2894) (end 147.066 81.0368) (width 0.25) (layer F.Cu) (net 15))
 (segment (start 151.8666 80.2894) (end 147.8134 80.2894) (width 0.25) (layer F.Cu) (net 15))
 (segment (start 147.066 82.16817) (end 147.200401 82.302571) (width 0.25) (layer F.Cu) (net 15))
 (segment (start 147.066 81.0368) (end 147.066 82.16817) (width 0.25) (layer F.Cu) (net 15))
 (segment (start 146.2532 91.93423) (end 146.2532 93.0656) (width 0.25) (layer F.Cu) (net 15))
 (segment (start 146.2532 87.34919) (end 146.2532 91.93423) (width 0.25) (layer F.Cu) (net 15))
 (segment (start 147.4978 86.10459) (end 146.2532 87.34919) (width 0.25) (layer F.Cu) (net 15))
 (segment (start 147.4978 82.59997) (end 147.4978 86.10459) (width 0.25) (layer F.Cu) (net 15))
 (segment (start 147.066 82.16817) (end 147.4978 82.59997) (width 0.25) (layer F.Cu) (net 15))
 (segment (start 149.5406 76.1492) (end 151.8012 78.4098) (width 0.25) (layer F.Cu) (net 17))
 (segment (start 154.887 78.4098) (end 156.7666 80.2894) (width 0.25) (layer F.Cu) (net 17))
 (segment (start 151.8012 78.4098) (end 154.887 78.4098) (width 0.25) (layer F.Cu) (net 17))
 (segment (start 156.016601 81.039399) (end 156.7666 80.2894) (width 0.25) (layer F.Cu) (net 17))
 (segment (start 152.5778 84.4782) (end 156.016601 81.039399) (width 0.25) (layer F.Cu) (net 17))
 (segment (start 152.5778 89.281) (end 152.5778 84.4782) (width 0.25) (layer F.Cu) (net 17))
 (segment (start 148.7932 93.0656) (end 152.5778 89.281) (width 0.25) (layer F.Cu) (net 17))
 (segment (start 131.3688 83.5406) (end 129.8956 82.0674) (width 0.25) (layer B.Cu) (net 13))
 (segment (start 131.5466 83.7184) (end 131.3688 83.5406) (width 0.25) (layer B.Cu) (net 13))
 (segment (start 131.688823 83.860623) (end 131.3688 83.5406) (width 0.25) (layer B.Cu) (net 13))
 (segment (start 139.0224 84.085022) (end 138.798001 83.860623) (width 0.25) (layer B.Cu) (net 13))
 (segment (start 138.798001 83.860623) (end 131.688823 83.860623) (width 0.25) (layer B.Cu) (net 13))
 (segment (start 142.352622 84.085022) (end 139.0224 84.085022) (width 0.25) (layer B.Cu) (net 13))
 (segment (start 143.7132 85.4456) (end 142.352622 84.085022) (width 0.25) (layer B.Cu) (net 13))
 (segment (start 128.7272 71.9328) (end 126.0856 74.5744) (width 0.25) (layer B.Cu) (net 1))
 (segment (start 133.4008 71.9328) (end 128.7272 71.9328) (width 0.25) (layer B.Cu) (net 1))
 (segment (start 134.7512 71.9328) (end 133.4008 71.9328) (width 0.25) (layer B.Cu) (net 1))
 (segment (start 144.454 81.6356) (end 134.7512 71.9328) (width 0.25) (layer B.Cu) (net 1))
 (segment (start 124.1044 90.1868) (end 125.9332 92.0156) (width 0.25) (layer F.Cu) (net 1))
 (segment (start 125.9332 92.0156) (end 125.9332 93.0656) (width 0.25) (layer F.Cu) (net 1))
 (segment (start 124.1044 76.5556) (end 124.1044 90.1868) (width 0.25) (layer F.Cu) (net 1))
 (segment (start 126.0856 74.5744) (end 124.1044 76.5556) (width 0.25) (layer F.Cu) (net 1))
 (segment (start 127.21697 82.0744) (end 126.0856 82.0744) (width 0.25) (layer F.Cu) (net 27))
 (segment (start 129.7432 84.60063) (end 127.21697 82.0744) (width 0.25) (layer F.Cu) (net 27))
 (segment (start 129.7432 93.8022) (end 129.7432 84.60063) (width 0.25) (layer F.Cu) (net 27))
 (segment (start 130.7846 94.8436) (end 129.7432 93.8022) (width 0.25) (layer F.Cu) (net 27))
 (segment (start 130.7846 108.8136) (end 130.7846 94.8436) (width 0.25) (layer F.Cu) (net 27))
 (segment (start 139.954 68.6562) (end 136.6774 71.9328) (width 0.25) (layer F.Cu) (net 28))
 (segment (start 141.475208 68.6562) (end 141.4272 68.6562) (width 0.25) (layer F.Cu) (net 28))
 (segment (start 142.7988 68.6054) (end 141.526008 68.6054) (width 0.25) (layer F.Cu) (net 28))
 (segment (start 141.526008 68.6054) (end 141.475208 68.6562) (width 0.25) (layer F.Cu) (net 28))
 (segment (start 141.4272 68.6562) (end 139.954 68.6562) (width 0.25) (layer F.Cu) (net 28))
 (segment (start 141.605 68.6562) (end 141.4272 68.6562) (width 0.25) (layer F.Cu) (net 28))
 (segment (start 138.6332 85.4456) (end 137.498234 84.310634) (width 0.25) (layer B.Cu) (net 16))
 (segment (start 137.498234 84.310634) (end 125.403164 84.310634) (width 0.25) (layer B.Cu) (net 16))
 (segment (start 125.403164 84.310634) (end 124.808199 84.905599) (width 0.25) (layer B.Cu) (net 16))
 (segment (start 126.238 109.887801) (end 124.808199 108.458) (width 0.25) (layer B.Cu) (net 16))
 (segment (start 126.238 111.76) (end 126.238 109.887801) (width 0.25) (layer B.Cu) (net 16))
 (segment (start 124.808199 84.905599) (end 124.808199 108.458) (width 0.25) (layer B.Cu) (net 16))
 (segment (start 158.158 111.76) (end 159.258 111.76) (width 0.25) (layer B.Cu) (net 18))
 (segment (start 139.758201 93.360201) (end 158.158 111.76) (width 0.25) (layer B.Cu) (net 18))
 (segment (start 139.758201 89.110601) (end 139.758201 93.360201) (width 0.25) (layer B.Cu) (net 18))
 (segment (start 136.0932 85.4456) (end 139.758201 89.110601) (width 0.25) (layer B.Cu) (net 18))
 (segment (start 131.634599 113.043601) (end 130.7846 113.8936) (width 0.25) (layer B.Cu) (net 3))
 (segment (start 132.2324 112.4458) (end 131.634599 113.043601) (width 0.25) (layer B.Cu) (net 3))
 (segment (start 131.519596 107.414996) (end 132.2324 108.1278) (width 0.25) (layer B.Cu) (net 3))
 (segment (start 132.2324 108.1278) (end 132.2324 112.4458) (width 0.25) (layer B.Cu) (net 3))
 (segment (start 131.519596 96.111996) (end 131.519596 107.414996) (width 0.25) (layer B.Cu) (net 3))
 (segment (start 128.4732 93.0656) (end 131.519596 96.111996) (width 0.25) (layer B.Cu) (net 3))
 (segment (start 131.813199 93.865599) (end 131.0132 93.0656) (width 0.25) (layer F.Cu) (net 5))
 (segment (start 132.4102 94.4626) (end 131.813199 93.865599) (width 0.25) (layer F.Cu) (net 5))
 (segment (start 132.4102 109.728) (end 132.4102 94.4626) (width 0.25) (layer F.Cu) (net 5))
 (segment (start 130.7846 111.3536) (end 132.4102 109.728) (width 0.25) (layer F.Cu) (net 5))
 (segment (start 137.1854 82.0928) (end 136.6774 82.0928) (width 0.25) (layer B.Cu) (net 20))
 (segment (start 133.5532 85.217) (end 133.5532 85.4456) (width 0.25) (layer F.Cu) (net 20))
 (segment (start 136.6774 82.0928) (end 133.5532 85.217) (width 0.25) (layer F.Cu) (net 20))
 (segment (start 139.3952 83.185) (end 145.034 83.185) (width 0.25) (layer B.Cu) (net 20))
 (segment (start 145.034 83.185) (end 145.796 82.423) (width 0.25) (layer B.Cu) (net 20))
 (segment (start 138.303 82.0928) (end 139.3952 83.185) (width 0.25) (layer B.Cu) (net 20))
 (segment (start 136.6774 82.0928) (end 138.303 82.0928) (width 0.25) (layer B.Cu) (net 20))
 (segment (start 145.796 78.931802) (end 145.796 80.6958) (width 0.25) (layer B.Cu) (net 20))
 (segment (start 145.796 82.3214) (end 145.796 80.6958) (width 0.25) (layer B.Cu) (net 20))
 (segment (start 145.796 82.423) (end 145.796 82.3214) (width 0.25) (layer B.Cu) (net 20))
 (segment (start 149.9108 67.183) (end 149.9108 71.639802) (width 0.25) (layer B.Cu) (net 20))
 (segment (start 149.9108 71.639802) (end 145.669 75.881602) (width 0.25) (layer B.Cu) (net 20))
 (segment (start 145.669 75.881602) (end 145.796 76.008602) (width 0.25) (layer B.Cu) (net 20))
 (segment (start 145.796 76.008602) (end 145.796 82.3214) (width 0.25) (layer B.Cu) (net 20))
 (segment (start 131.990199 70.807799) (end 128.770599 74.027399) (width 0.25) (layer F.Cu) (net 22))
 (segment (start 128.770599 75.107401) (end 131.813199 78.150001) (width 0.25) (layer F.Cu) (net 22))
 (segment (start 137.165991 70.807799) (end 131.990199 70.807799) (width 0.25) (layer F.Cu) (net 22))
 (segment (start 131.813199 84.645601) (end 131.0132 85.4456) (width 0.25) (layer F.Cu) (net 22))
 (segment (start 140.79079 67.183) (end 137.165991 70.807799) (width 0.25) (layer F.Cu) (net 22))
 (segment (start 146.7866 67.183) (end 140.79079 67.183) (width 0.25) (layer F.Cu) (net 22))
 (segment (start 131.813199 78.150001) (end 131.813199 84.645601) (width 0.25) (layer F.Cu) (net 22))
 (segment (start 128.770599 74.027399) (end 128.770599 75.107401) (width 0.25) (layer F.Cu) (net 22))
 (segment (start 151.4602 71.8566) (end 146.7866 67.183) (width 0.25) (layer F.Cu) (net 22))
 (segment (start 152.1968 71.8566) (end 151.4602 71.8566) (width 0.25) (layer F.Cu) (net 22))
 (segment (start 158.6968 71.374) (end 158.6968 75.874) (width 0.25) (layer F.Cu) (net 29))
 (segment (start 139.954 75.1356) (end 144.454 75.1356) (width 0.25) (layer F.Cu) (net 30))
 (segment (start 133.5532 93.0656) (end 136.6774 96.1898) (width 0.25) (layer F.Cu) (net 7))
 (segment (start 138.2268 96.1898) (end 141.8844 99.8474) (width 0.25) (layer F.Cu) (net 7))
 (segment (start 136.6774 96.1898) (end 138.2268 96.1898) (width 0.25) (layer F.Cu) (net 7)))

